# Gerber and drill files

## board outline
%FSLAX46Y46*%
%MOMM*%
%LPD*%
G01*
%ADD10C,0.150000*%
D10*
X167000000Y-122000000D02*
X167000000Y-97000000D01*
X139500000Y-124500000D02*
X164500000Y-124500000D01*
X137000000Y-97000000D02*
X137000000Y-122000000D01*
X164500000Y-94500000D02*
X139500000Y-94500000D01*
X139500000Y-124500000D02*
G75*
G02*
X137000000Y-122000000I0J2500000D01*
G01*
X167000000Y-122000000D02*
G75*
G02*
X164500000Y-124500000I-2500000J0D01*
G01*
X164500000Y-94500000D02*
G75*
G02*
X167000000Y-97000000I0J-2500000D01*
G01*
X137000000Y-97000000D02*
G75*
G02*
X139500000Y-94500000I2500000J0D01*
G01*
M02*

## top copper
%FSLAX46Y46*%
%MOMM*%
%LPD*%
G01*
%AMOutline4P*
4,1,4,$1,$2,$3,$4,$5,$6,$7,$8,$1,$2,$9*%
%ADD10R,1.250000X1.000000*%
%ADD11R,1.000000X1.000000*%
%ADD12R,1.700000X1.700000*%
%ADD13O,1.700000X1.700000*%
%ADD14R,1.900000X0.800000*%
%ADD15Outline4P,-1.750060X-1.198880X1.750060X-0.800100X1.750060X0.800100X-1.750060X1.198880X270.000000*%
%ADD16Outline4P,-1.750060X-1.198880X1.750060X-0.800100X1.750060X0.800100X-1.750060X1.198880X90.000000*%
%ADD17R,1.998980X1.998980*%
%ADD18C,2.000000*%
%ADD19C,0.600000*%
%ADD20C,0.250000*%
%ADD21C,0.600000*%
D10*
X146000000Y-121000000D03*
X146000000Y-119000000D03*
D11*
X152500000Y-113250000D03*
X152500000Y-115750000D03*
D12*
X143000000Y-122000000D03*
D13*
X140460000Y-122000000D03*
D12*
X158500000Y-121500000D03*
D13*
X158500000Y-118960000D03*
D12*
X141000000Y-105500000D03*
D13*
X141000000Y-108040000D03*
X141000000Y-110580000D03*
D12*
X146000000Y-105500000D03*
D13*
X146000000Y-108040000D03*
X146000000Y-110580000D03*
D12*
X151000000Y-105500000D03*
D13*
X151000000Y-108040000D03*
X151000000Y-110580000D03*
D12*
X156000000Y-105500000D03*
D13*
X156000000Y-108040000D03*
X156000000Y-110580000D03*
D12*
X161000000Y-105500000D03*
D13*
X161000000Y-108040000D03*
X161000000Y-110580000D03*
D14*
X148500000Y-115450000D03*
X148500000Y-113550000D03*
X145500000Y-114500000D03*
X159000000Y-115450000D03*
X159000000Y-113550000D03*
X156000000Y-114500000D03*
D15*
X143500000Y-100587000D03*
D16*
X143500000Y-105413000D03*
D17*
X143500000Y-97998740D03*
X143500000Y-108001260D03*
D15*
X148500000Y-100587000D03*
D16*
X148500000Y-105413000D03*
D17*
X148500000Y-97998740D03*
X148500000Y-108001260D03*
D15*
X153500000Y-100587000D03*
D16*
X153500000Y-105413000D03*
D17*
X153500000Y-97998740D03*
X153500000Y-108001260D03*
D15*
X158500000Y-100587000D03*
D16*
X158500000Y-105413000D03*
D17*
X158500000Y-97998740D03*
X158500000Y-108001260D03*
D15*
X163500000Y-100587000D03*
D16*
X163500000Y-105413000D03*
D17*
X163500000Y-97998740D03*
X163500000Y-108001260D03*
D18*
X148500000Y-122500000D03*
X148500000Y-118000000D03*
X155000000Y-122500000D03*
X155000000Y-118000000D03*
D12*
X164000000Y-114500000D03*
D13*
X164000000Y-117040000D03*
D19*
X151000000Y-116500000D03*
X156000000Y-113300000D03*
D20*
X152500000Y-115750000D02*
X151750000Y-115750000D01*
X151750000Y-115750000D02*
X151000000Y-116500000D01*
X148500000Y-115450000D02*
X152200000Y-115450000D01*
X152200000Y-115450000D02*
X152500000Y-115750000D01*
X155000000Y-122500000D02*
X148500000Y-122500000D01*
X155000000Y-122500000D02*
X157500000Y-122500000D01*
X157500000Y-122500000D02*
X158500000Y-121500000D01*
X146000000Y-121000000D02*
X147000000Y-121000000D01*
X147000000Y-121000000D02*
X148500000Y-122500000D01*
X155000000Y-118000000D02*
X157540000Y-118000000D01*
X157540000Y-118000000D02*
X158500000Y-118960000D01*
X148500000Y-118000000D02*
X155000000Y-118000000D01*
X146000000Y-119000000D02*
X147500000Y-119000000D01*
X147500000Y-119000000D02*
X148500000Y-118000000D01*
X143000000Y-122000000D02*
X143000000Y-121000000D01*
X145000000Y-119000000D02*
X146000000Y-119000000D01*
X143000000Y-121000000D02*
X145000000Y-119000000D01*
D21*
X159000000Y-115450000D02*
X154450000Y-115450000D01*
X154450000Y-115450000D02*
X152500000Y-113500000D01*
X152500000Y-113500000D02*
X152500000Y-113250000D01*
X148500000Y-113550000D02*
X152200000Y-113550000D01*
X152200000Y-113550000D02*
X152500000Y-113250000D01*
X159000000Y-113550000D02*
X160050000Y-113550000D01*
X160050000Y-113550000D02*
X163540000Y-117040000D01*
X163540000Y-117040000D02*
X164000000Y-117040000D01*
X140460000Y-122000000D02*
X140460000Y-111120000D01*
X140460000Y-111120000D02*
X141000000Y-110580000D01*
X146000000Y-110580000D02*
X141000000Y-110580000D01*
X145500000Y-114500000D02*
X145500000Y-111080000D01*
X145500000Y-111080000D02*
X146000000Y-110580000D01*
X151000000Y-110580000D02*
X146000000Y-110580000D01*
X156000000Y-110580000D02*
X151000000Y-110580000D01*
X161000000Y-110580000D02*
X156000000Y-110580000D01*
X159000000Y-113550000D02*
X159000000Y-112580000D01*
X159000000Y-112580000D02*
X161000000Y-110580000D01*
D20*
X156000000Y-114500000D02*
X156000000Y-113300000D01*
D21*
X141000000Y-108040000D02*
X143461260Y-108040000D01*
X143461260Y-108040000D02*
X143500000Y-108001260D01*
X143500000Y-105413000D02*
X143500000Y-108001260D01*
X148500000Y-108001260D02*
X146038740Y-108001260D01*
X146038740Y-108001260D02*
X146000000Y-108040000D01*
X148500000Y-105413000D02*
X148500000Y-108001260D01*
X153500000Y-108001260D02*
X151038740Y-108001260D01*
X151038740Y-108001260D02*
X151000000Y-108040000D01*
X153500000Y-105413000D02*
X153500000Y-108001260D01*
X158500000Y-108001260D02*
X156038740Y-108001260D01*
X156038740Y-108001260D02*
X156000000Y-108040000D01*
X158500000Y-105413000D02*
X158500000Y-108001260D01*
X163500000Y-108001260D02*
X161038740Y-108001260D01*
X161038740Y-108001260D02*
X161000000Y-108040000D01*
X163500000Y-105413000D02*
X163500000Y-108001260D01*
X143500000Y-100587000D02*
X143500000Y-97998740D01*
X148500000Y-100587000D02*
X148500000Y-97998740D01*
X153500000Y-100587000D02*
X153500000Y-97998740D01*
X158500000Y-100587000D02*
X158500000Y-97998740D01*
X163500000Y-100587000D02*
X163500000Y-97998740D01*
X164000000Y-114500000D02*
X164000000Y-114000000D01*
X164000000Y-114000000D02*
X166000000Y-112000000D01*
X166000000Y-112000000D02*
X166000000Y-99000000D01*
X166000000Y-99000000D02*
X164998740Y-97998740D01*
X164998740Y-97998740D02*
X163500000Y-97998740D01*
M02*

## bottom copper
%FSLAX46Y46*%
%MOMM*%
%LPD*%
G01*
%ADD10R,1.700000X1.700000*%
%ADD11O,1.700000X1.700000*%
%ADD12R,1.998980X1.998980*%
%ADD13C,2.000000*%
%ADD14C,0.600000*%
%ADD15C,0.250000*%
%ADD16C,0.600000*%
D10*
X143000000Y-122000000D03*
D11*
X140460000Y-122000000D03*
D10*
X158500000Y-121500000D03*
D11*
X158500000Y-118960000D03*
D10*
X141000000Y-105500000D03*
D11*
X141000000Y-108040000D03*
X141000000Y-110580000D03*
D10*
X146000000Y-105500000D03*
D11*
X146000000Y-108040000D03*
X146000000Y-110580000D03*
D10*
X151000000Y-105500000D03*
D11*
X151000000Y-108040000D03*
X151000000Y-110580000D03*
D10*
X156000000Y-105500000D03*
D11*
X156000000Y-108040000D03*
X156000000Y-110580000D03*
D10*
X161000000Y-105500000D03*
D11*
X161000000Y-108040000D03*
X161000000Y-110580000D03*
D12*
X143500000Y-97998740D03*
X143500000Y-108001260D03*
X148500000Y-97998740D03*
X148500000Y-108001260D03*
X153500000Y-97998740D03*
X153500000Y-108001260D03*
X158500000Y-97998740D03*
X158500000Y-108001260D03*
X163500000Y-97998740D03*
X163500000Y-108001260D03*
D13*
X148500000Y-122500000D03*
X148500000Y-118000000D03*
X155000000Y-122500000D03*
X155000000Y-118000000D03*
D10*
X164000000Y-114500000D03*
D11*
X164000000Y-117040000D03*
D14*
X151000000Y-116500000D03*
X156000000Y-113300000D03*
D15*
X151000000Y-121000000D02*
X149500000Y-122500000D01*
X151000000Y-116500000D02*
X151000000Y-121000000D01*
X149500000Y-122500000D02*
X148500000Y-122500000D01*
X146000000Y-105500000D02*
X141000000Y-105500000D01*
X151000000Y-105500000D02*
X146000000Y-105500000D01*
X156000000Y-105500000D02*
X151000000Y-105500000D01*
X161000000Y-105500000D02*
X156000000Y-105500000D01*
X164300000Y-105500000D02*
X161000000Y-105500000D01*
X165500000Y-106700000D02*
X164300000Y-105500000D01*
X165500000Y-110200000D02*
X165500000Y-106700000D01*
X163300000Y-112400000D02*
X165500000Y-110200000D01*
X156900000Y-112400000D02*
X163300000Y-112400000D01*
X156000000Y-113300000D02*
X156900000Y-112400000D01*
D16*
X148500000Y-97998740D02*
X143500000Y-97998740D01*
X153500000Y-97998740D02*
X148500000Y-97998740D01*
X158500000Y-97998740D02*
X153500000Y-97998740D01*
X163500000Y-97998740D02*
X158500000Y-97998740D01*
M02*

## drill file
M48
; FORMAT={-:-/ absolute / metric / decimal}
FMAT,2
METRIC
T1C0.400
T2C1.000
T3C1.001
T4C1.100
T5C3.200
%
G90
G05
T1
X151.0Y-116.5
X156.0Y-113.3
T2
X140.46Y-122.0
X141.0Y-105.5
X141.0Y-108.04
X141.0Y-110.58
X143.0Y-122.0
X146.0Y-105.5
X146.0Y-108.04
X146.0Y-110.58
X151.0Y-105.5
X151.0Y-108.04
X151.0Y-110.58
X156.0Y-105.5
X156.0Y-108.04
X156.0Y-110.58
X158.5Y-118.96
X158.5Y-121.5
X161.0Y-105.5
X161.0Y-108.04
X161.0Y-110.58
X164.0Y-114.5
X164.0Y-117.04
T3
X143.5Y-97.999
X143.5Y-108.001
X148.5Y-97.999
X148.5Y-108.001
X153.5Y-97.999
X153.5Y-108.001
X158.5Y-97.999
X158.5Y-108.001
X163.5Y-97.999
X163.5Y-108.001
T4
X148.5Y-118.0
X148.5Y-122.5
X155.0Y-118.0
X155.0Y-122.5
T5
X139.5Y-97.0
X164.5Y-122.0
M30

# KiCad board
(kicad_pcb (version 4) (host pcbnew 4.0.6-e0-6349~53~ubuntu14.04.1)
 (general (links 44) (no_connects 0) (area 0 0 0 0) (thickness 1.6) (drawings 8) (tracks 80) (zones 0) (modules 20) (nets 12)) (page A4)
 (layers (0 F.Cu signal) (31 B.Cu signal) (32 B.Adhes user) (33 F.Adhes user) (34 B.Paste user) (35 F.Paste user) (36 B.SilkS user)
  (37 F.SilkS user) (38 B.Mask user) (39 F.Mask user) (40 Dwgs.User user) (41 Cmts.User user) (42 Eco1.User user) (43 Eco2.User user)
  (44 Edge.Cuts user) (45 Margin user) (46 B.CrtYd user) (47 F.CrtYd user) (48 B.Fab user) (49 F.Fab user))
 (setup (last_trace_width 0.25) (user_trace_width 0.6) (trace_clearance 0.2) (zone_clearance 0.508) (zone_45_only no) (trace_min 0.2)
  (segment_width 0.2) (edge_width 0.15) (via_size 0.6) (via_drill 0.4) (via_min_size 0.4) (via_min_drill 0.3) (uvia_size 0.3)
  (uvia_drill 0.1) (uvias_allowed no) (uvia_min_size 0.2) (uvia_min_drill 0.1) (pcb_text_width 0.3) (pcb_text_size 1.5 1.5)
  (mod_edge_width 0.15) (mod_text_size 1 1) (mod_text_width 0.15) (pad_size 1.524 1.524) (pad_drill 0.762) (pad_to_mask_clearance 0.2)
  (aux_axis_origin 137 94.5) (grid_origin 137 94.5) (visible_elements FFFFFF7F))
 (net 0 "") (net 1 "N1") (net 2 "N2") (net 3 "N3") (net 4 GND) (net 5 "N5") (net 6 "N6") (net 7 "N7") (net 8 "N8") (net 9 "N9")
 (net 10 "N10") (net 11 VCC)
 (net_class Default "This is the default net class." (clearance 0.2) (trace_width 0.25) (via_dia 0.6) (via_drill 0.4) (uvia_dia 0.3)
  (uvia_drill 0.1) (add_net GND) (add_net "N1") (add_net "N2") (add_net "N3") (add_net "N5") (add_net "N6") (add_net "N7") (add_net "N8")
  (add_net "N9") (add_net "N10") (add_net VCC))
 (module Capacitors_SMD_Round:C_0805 (layer F.Cu) (at 146 120 90)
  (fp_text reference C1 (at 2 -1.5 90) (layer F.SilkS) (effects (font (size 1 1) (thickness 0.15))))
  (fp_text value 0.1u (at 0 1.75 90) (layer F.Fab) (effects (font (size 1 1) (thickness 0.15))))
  (pad 1 smd rect (at -1 0 90) (size 1 1.25) (layers F.Cu F.Paste F.Mask) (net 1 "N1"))
  (pad 2 smd rect (at 1 0 90) (size 1 1.25) (layers F.Cu F.Paste F.Mask) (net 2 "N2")))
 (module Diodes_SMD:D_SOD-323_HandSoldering (layer F.Cu) (at 152.5 114.5 270)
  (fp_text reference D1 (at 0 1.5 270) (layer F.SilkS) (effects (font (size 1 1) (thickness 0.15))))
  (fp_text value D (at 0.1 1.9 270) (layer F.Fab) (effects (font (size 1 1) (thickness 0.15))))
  (pad 1 smd rect (at -1.25 0 270) (size 1 1) (layers F.Cu F.Paste F.Mask) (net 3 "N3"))
  (pad 2 smd rect (at 1.25 0 270) (size 1 1) (layers F.Cu F.Paste F.Mask) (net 1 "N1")))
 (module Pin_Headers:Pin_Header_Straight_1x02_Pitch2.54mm (layer F.Cu) (at 143 122 270)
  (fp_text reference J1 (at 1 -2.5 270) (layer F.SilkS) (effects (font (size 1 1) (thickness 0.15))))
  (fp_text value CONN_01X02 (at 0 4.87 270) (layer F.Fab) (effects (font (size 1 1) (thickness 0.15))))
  (pad 1 thru_hole rect (at 0 0 270) (size 1.7 1.7) (drill 1) (layers *.Cu *.Mask) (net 2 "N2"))
  (pad 2 thru_hole oval (at 0 2.54 270) (size 1.7 1.7) (drill 1) (layers *.Cu *.Mask) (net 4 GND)))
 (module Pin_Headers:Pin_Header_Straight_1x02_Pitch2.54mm (layer F.Cu) (at 158.5 121.5 180)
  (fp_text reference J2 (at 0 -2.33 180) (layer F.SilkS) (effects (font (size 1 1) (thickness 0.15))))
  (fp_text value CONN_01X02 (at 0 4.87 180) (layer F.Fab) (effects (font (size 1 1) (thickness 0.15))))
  (pad 1 thru_hole rect (at 0 0 180) (size 1.7 1.7) (drill 1) (layers *.Cu *.Mask) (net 1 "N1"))
  (pad 2 thru_hole oval (at 0 2.54 180) (size 1.7 1.7) (drill 1) (layers *.Cu *.Mask) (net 2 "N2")))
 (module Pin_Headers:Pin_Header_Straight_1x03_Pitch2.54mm (layer F.Cu) (at 141 105.5)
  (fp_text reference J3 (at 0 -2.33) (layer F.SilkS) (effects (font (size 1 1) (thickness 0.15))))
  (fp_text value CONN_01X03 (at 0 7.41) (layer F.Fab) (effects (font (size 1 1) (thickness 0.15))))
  (pad 1 thru_hole rect (at 0 0) (size 1.7 1.7) (drill 1) (layers *.Cu *.Mask) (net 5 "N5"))
  (pad 2 thru_hole oval (at 0 2.54) (size 1.7 1.7) (drill 1) (layers *.Cu *.Mask) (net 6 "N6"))
  (pad 3 thru_hole oval (at 0 5.08) (size 1.7 1.7) (drill 1) (layers *.Cu *.Mask) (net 4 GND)))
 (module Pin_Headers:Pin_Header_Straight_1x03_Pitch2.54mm (layer F.Cu) (at 146 105.5)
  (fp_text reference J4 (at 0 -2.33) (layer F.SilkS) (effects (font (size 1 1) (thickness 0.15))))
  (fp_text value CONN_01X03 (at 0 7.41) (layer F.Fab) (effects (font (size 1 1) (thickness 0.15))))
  (pad 1 thru_hole rect (at 0 0) (size 1.7 1.7) (drill 1) (layers *.Cu *.Mask) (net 5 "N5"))
  (pad 2 thru_hole oval (at 0 2.54) (size 1.7 1.7) (drill 1) (layers *.Cu *.Mask) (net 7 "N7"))
  (pad 3 thru_hole oval (at 0 5.08) (size 1.7 1.7) (drill 1) (layers *.Cu *.Mask) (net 4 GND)))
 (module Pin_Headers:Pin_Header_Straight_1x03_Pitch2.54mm (layer F.Cu) (at 151 105.5)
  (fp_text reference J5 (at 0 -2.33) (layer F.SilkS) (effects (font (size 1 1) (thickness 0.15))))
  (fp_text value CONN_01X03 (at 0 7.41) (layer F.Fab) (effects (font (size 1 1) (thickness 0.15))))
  (pad 1 thru_hole rect (at 0 0) (size 1.7 1.7) (drill 1) (layers *.Cu *.Mask) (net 5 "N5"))
  (pad 2 thru_hole oval (at 0 2.54) (size 1.7 1.7) (drill 1) (layers *.Cu *.Mask) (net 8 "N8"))
  (pad 3 thru_hole oval (at 0 5.08) (size 1.7 1.7) (drill 1) (layers *.Cu *.Mask) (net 4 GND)))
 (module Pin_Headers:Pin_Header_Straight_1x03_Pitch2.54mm (layer F.Cu) (at 156 105.5)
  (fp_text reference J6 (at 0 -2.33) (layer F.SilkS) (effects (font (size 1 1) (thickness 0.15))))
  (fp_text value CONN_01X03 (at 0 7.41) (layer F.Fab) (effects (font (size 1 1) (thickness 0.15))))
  (pad 1 thru_hole rect (at 0 0) (size 1.7 1.7) (drill 1) (layers *.Cu *.Mask) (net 5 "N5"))
  (pad 2 thru_hole oval (at 0 2.54) (size 1.7 1.7) (drill 1) (layers *.Cu *.Mask) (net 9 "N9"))
  (pad 3 thru_hole oval (at 0 5.08) (size 1.7 1.7) (drill 1) (layers *.Cu *.Mask) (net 4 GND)))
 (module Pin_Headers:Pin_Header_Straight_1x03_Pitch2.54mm (layer F.Cu) (at 161 105.5)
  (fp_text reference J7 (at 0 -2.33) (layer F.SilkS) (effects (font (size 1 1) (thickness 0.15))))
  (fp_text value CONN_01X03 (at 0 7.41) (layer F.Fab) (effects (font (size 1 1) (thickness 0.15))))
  (pad 1 thru_hole rect (at 0 0) (size 1.7 1.7) (drill 1) (layers *.Cu *.Mask) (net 5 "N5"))
  (pad 2 thru_hole oval (at 0 2.54) (size 1.7 1.7) (drill 1) (layers *.Cu *.Mask) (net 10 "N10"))
  (pad 3 thru_hole oval (at 0 5.08) (size 1.7 1.7) (drill 1) (layers *.Cu *.Mask) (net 4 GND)))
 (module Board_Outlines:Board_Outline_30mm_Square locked (layer F.Cu) (at 137 94.5)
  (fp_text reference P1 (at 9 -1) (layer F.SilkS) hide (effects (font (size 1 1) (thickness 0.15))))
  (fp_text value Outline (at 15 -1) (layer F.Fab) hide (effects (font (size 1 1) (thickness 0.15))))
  (fp_line (start 30 27.5) (end 30 2.5) (layer Edge.Cuts) (width 0.15))
  (fp_line (start 2.5 30) (end 27.5 30) (layer Edge.Cuts) (width 0.15))
  (fp_line (start 0 2.5) (end 0 27.5) (layer Edge.Cuts) (width 0.15))
  (fp_line (start 27.5 0) (end 2.5 0) (layer Edge.Cuts) (width 0.15))
  (fp_arc (start 2.5 27.5) (end 2.5 30) (angle 90) (layer Edge.Cuts) (width 0.15))
  (fp_arc (start 27.5 27.5) (end 30 27.5) (angle 90) (layer Edge.Cuts) (width 0.15))
  (fp_arc (start 27.5 2.5) (end 27.5 0) (angle 90) (layer Edge.Cuts) (width 0.15))
  (fp_arc (start 2.5 2.5) (end 0 2.5) (angle 90) (layer Edge.Cuts) (width 0.15))
  (pad "" np_thru_hole circle (at 2.5 2.5) (size 3.2 3.2) (drill 3.2) (layers *.Cu *.Mask))
  (pad "" np_thru_hole circle (at 27.5 27.5) (size 3.2 3.2) (drill 3.2) (layers *.Cu *.Mask)))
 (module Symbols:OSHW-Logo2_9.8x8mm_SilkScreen (layer B.Cu) (at 142.5 116)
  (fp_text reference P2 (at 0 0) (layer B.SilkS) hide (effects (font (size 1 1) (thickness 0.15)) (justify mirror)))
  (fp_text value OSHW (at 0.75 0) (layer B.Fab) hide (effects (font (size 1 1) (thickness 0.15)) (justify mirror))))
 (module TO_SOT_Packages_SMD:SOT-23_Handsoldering (layer F.Cu) (at 147 114.5 180)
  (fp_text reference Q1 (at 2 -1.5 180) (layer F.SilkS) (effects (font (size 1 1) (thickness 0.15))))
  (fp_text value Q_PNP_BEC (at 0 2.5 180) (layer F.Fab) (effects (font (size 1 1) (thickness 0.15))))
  (pad 1 smd rect (at -1.5 -0.95 180) (size 1.9 0.8) (layers F.Cu F.Paste F.Mask) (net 1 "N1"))
  (pad 2 smd rect (at -1.5 0.95 180) (size 1.9 0.8) (layers F.Cu F.Paste F.Mask) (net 3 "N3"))
  (pad 3 smd rect (at 1.5 0 180) (size 1.9 0.8) (layers F.Cu F.Paste F.Mask) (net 4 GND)))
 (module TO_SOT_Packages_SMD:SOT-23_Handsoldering (layer F.Cu) (at 157.5 114.5 180)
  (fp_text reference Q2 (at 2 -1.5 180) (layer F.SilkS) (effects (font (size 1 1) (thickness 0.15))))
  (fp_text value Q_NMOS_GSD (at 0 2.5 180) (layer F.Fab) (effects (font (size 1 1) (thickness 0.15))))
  (pad 1 smd rect (at -1.5 -0.95 180) (size 1.9 0.8) (layers F.Cu F.Paste F.Mask) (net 3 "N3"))
  (pad 2 smd rect (at -1.5 0.95 180) (size 1.9 0.8) (layers F.Cu F.Paste F.Mask) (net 4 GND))
  (pad 3 smd rect (at 1.5 0 180) (size 1.9 0.8) (layers F.Cu F.Paste F.Mask) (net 5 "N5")))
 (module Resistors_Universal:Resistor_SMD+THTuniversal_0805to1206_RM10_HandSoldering (layer F.Cu) (at 143.5 103 270)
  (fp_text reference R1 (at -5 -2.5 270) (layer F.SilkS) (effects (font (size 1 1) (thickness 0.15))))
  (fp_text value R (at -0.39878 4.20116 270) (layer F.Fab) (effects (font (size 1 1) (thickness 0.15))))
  (pad 1 smd trapezoid (at -2.413 0 270) (size 3.50012 1.99898) (rect_delta 0.39878 0) (layers F.Cu F.Paste F.Mask) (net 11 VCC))
  (pad 2 smd trapezoid (at 2.413 0 90) (size 3.50012 1.99898) (rect_delta 0.39878 0) (layers F.Cu F.Paste F.Mask) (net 6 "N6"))
  (pad 1 thru_hole rect (at -5.00126 0 90) (size 1.99898 1.99898) (drill 1.00076) (layers *.Cu *.Mask) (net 11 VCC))
  (pad 2 thru_hole rect (at 5.00126 0 90) (size 1.99898 1.99898) (drill 1.00076) (layers *.Cu *.Mask) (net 6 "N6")))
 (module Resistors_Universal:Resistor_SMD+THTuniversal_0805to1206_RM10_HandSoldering (layer F.Cu) (at 148.5 103 270)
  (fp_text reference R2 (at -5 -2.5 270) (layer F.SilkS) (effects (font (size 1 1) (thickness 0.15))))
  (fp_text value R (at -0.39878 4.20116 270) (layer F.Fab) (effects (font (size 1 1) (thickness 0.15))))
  (pad 1 smd trapezoid (at -2.413 0 270) (size 3.50012 1.99898) (rect_delta 0.39878 0) (layers F.Cu F.Paste F.Mask) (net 11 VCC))
  (pad 2 smd trapezoid (at 2.413 0 90) (size 3.50012 1.99898) (rect_delta 0.39878 0) (layers F.Cu F.Paste F.Mask) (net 7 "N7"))
  (pad 1 thru_hole rect (at -5.00126 0 90) (size 1.99898 1.99898) (drill 1.00076) (layers *.Cu *.Mask) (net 11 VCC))
  (pad 2 thru_hole rect (at 5.00126 0 90) (size 1.99898 1.99898) (drill 1.00076) (layers *.Cu *.Mask) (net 7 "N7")))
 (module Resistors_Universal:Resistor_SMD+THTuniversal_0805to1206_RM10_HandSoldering (layer F.Cu) (at 153.5 103 270)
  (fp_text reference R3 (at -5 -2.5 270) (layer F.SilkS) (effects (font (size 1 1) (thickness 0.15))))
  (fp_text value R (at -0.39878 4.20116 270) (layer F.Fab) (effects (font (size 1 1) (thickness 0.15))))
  (pad 1 smd trapezoid (at -2.413 0 270) (size 3.50012 1.99898) (rect_delta 0.39878 0) (layers F.Cu F.Paste F.Mask) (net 11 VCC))
  (pad 2 smd trapezoid (at 2.413 0 90) (size 3.50012 1.99898) (rect_delta 0.39878 0) (layers F.Cu F.Paste F.Mask) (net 8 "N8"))
  (pad 1 thru_hole rect (at -5.00126 0 90) (size 1.99898 1.99898) (drill 1.00076) (layers *.Cu *.Mask) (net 11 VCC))
  (pad 2 thru_hole rect (at 5.00126 0 90) (size 1.99898 1.99898) (drill 1.00076) (layers *.Cu *.Mask) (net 8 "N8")))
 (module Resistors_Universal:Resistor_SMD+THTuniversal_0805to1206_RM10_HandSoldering (layer F.Cu) (at 158.5 103 270)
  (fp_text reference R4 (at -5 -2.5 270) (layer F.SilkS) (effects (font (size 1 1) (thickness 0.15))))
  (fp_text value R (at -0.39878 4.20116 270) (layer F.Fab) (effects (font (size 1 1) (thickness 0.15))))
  (pad 1 smd trapezoid (at -2.413 0 270) (size 3.50012 1.99898) (rect_delta 0.39878 0) (layers F.Cu F.Paste F.Mask) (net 11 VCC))
  (pad 2 smd trapezoid (at 2.413 0 90) (size 3.50012 1.99898) (rect_delta 0.39878 0) (layers F.Cu F.Paste F.Mask) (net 9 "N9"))
  (pad 1 thru_hole rect (at -5.00126 0 90) (size 1.99898 1.99898) (drill 1.00076) (layers *.Cu *.Mask) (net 11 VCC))
  (pad 2 thru_hole rect (at 5.00126 0 90) (size 1.99898 1.99898) (drill 1.00076) (layers *.Cu *.Mask) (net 9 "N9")))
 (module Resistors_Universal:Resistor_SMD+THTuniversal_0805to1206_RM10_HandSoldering (layer F.Cu) (at 163.5 103 270)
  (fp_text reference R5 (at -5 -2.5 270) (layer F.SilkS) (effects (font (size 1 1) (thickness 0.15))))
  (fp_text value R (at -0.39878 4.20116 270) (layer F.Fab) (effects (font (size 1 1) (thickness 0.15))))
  (pad 1 smd trapezoid (at -2.413 0 270) (size 3.50012 1.99898) (rect_delta 0.39878 0) (layers F.Cu F.Paste F.Mask) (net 11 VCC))
  (pad 2 smd trapezoid (at 2.413 0 90) (size 3.50012 1.99898) (rect_delta 0.39878 0) (layers F.Cu F.Paste F.Mask) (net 10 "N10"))
  (pad 1 thru_hole rect (at -5.00126 0 90) (size 1.99898 1.99898) (drill 1.00076) (layers *.Cu *.Mask) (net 11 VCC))
  (pad 2 thru_hole rect (at 5.00126 0 90) (size 1.99898 1.99898) (drill 1.00076) (layers *.Cu *.Mask) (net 10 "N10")))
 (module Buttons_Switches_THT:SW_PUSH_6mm (layer F.Cu) (at 148.5 118)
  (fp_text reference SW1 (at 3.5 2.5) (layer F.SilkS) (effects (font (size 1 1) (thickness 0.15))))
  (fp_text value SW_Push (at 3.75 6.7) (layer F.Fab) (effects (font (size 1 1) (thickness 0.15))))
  (pad 2 thru_hole circle (at 0 4.5 90) (size 2 2) (drill 1.1) (layers *.Cu *.Mask) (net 1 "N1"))
  (pad 1 thru_hole circle (at 0 0 90) (size 2 2) (drill 1.1) (layers *.Cu *.Mask) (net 2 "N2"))
  (pad 2 thru_hole circle (at 6.5 4.5 90) (size 2 2) (drill 1.1) (layers *.Cu *.Mask) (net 1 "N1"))
  (pad 1 thru_hole circle (at 6.5 0 90) (size 2 2) (drill 1.1) (layers *.Cu *.Mask) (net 2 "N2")))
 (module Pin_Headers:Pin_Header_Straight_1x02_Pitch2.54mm (layer F.Cu) (at 164 114.5)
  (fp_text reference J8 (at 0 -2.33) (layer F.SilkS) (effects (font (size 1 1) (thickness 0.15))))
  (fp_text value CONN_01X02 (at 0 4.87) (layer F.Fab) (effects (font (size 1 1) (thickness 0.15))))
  (pad 1 thru_hole rect (at 0 0) (size 1.7 1.7) (drill 1) (layers *.Cu *.Mask) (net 11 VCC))
  (pad 2 thru_hole oval (at 0 2.54) (size 1.7 1.7) (drill 1) (layers *.Cu *.Mask) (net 4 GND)))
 (segment (start 152.5 115.75) (end 151.75 115.75) (width 0.25) (layer F.Cu) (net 1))
 (segment (start 151 121) (end 149.5 122.5) (width 0.25) (layer B.Cu) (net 1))
 (segment (start 151 116.5) (end 151 121) (width 0.25) (layer B.Cu) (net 1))
 (via (at 151 116.5) (size 0.6) (drill 0.4) (layers F.Cu B.Cu) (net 1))
 (segment (start 151.75 115.75) (end 151 116.5) (width 0.25) (layer F.Cu) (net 1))
 (segment (start 149.5 122.5) (end 148.5 122.5) (width 0.25) (layer B.Cu) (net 1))
 (segment (start 148.5 115.45) (end 152.2 115.45) (width 0.25) (layer F.Cu) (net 1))
 (segment (start 152.2 115.45) (end 152.5 115.75) (width 0.25) (layer F.Cu) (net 1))
 (segment (start 155 122.5) (end 148.5 122.5) (width 0.25) (layer F.Cu) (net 1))
 (segment (start 155 122.5) (end 157.5 122.5) (width 0.25) (layer F.Cu) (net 1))
 (segment (start 157.5 122.5) (end 158.5 121.5) (width 0.25) (layer F.Cu) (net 1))
 (segment (start 146 121) (end 147 121) (width 0.25) (layer F.Cu) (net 1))
 (segment (start 147 121) (end 148.5 122.5) (width 0.25) (layer F.Cu) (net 1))
 (segment (start 155 118) (end 157.54 118) (width 0.25) (layer F.Cu) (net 2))
 (segment (start 157.54 118) (end 158.5 118.96) (width 0.25) (layer F.Cu) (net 2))
 (segment (start 148.5 118) (end 155 118) (width 0.25) (layer F.Cu) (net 2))
 (segment (start 146 119) (end 147.5 119) (width 0.25) (layer F.Cu) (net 2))
 (segment (start 147.5 119) (end 148.5 118) (width 0.25) (layer F.Cu) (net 2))
 (segment (start 143 122) (end 143 121) (width 0.25) (layer F.Cu) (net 2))
 (segment (start 145 119) (end 146 119) (width 0.25) (layer F.Cu) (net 2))
 (segment (start 143 121) (end 145 119) (width 0.25) (layer F.Cu) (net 2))
 (segment (start 159 115.45) (end 154.45 115.45) (width 0.6) (layer F.Cu) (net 3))
 (segment (start 154.45 115.45) (end 152.5 113.5) (width 0.6) (layer F.Cu) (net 3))
 (segment (start 152.5 113.5) (end 152.5 113.25) (width 0.6) (layer F.Cu) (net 3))
 (segment (start 148.5 113.55) (end 152.2 113.55) (width 0.6) (layer F.Cu) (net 3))
 (segment (start 152.2 113.55) (end 152.5 113.25) (width 0.6) (layer F.Cu) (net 3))
 (segment (start 159 113.55) (end 160.05 113.55) (width 0.6) (layer F.Cu) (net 4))
 (segment (start 160.05 113.55) (end 163.54 117.04) (width 0.6) (layer F.Cu) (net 4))
 (segment (start 163.54 117.04) (end 164 117.04) (width 0.6) (layer F.Cu) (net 4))
 (segment (start 140.46 122) (end 140.46 111.12) (width 0.6) (layer F.Cu) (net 4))
 (segment (start 140.46 111.12) (end 141 110.58) (width 0.6) (layer F.Cu) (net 4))
 (segment (start 146 110.58) (end 141 110.58) (width 0.6) (layer F.Cu) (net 4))
 (segment (start 145.5 114.5) (end 145.5 111.08) (width 0.6) (layer F.Cu) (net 4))
 (segment (start 145.5 111.08) (end 146 110.58) (width 0.6) (layer F.Cu) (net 4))
 (segment (start 151 110.58) (end 146 110.58) (width 0.6) (layer F.Cu) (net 4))
 (segment (start 156 110.58) (end 151 110.58) (width 0.6) (layer F.Cu) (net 4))
 (segment (start 161 110.58) (end 156 110.58) (width 0.6) (layer F.Cu) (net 4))
 (segment (start 159 113.55) (end 159 112.58) (width 0.6) (layer F.Cu) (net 4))
 (segment (start 159 112.58) (end 161 110.58) (width 0.6) (layer F.Cu) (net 4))
 (segment (start 146 105.5) (end 141 105.5) (width 0.25) (layer B.Cu) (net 5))
 (segment (start 151 105.5) (end 146 105.5) (width 0.25) (layer B.Cu) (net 5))
 (segment (start 156 105.5) (end 151 105.5) (width 0.25) (layer B.Cu) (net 5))
 (segment (start 161 105.5) (end 156 105.5) (width 0.25) (layer B.Cu) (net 5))
 (segment (start 156 114.5) (end 156 113.3) (width 0.25) (layer F.Cu) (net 5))
 (segment (start 164.3 105.5) (end 161 105.5) (width 0.25) (layer B.Cu) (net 5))
 (segment (start 165.5 106.7) (end 164.3 105.5) (width 0.25) (layer B.Cu) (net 5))
 (segment (start 165.5 110.2) (end 165.5 106.7) (width 0.25) (layer B.Cu) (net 5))
 (segment (start 163.3 112.4) (end 165.5 110.2) (width 0.25) (layer B.Cu) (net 5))
 (segment (start 156.9 112.4) (end 163.3 112.4) (width 0.25) (layer B.Cu) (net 5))
 (segment (start 156 113.3) (end 156.9 112.4) (width 0.25) (layer B.Cu) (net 5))
 (via (at 156 113.3) (size 0.6) (drill 0.4) (layers F.Cu B.Cu) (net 5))
 (segment (start 141 108.04) (end 143.46126 108.04) (width 0.6) (layer F.Cu) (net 6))
 (segment (start 143.46126 108.04) (end 143.5 108.00126) (width 0.6) (layer F.Cu) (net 6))
 (segment (start 143.5 105.413) (end 143.5 108.00126) (width 0.6) (layer F.Cu) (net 6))
 (segment (start 148.5 108.00126) (end 146.03874 108.00126) (width 0.6) (layer F.Cu) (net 7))
 (segment (start 146.03874 108.00126) (end 146 108.04) (width 0.6) (layer F.Cu) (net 7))
 (segment (start 148.5 105.413) (end 148.5 108.00126) (width 0.6) (layer F.Cu) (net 7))
 (segment (start 153.5 108.00126) (end 151.03874 108.00126) (width 0.6) (layer F.Cu) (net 8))
 (segment (start 151.03874 108.00126) (end 151 108.04) (width 0.6) (layer F.Cu) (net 8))
 (segment (start 153.5 105.413) (end 153.5 108.00126) (width 0.6) (layer F.Cu) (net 8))
 (segment (start 158.5 108.00126) (end 156.03874 108.00126) (width 0.6) (layer F.Cu) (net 9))
 (segment (start 156.03874 108.00126) (end 156 108.04) (width 0.6) (layer F.Cu) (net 9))
 (segment (start 158.5 105.413) (end 158.5 108.00126) (width 0.6) (layer F.Cu) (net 9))
 (segment (start 163.5 108.00126) (end 161.03874 108.00126) (width 0.6) (layer F.Cu) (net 10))
 (segment (start 161.03874 108.00126) (end 161 108.04) (width 0.6) (layer F.Cu) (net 10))
 (segment (start 163.5 105.413) (end 163.5 108.00126) (width 0.6) (layer F.Cu) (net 10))
 (segment (start 143.5 100.587) (end 143.5 97.99874) (width 0.6) (layer F.Cu) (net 11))
 (segment (start 148.5 100.587) (end 148.5 97.99874) (width 0.6) (layer F.Cu) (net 11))
 (segment (start 153.5 100.587) (end 153.5 97.99874) (width 0.6) (layer F.Cu) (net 11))
 (segment (start 158.5 100.587) (end 158.5 97.99874) (width 0.6) (layer F.Cu) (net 11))
 (segment (start 163.5 100.587) (end 163.5 97.99874) (width 0.6) (layer F.Cu) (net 11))
 (segment (start 164 114.5) (end 164 114) (width 0.6) (layer F.Cu) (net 11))
 (segment (start 164 114) (end 166 112) (width 0.6) (layer F.Cu) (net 11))
 (segment (start 166 112) (end 166 99) (width 0.6) (layer F.Cu) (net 11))
 (segment (start 166 99) (end 164.99874 97.99874) (width 0.6) (layer F.Cu) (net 11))
 (segment (start 164.99874 97.99874) (end 163.5 97.99874) (width 0.6) (layer F.Cu) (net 11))
 (segment (start 148.5 97.99874) (end 143.5 97.99874) (width 0.6) (layer B.Cu) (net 11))
 (segment (start 153.5 97.99874) (end 148.5 97.99874) (width 0.6) (layer B.Cu) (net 11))
 (segment (start 158.5 97.99874) (end 153.5 97.99874) (width 0.6) (layer B.Cu) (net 11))
 (segment (start 163.5 97.99874) (end 158.5 97.99874) (width 0.6) (layer B.Cu) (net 11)))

